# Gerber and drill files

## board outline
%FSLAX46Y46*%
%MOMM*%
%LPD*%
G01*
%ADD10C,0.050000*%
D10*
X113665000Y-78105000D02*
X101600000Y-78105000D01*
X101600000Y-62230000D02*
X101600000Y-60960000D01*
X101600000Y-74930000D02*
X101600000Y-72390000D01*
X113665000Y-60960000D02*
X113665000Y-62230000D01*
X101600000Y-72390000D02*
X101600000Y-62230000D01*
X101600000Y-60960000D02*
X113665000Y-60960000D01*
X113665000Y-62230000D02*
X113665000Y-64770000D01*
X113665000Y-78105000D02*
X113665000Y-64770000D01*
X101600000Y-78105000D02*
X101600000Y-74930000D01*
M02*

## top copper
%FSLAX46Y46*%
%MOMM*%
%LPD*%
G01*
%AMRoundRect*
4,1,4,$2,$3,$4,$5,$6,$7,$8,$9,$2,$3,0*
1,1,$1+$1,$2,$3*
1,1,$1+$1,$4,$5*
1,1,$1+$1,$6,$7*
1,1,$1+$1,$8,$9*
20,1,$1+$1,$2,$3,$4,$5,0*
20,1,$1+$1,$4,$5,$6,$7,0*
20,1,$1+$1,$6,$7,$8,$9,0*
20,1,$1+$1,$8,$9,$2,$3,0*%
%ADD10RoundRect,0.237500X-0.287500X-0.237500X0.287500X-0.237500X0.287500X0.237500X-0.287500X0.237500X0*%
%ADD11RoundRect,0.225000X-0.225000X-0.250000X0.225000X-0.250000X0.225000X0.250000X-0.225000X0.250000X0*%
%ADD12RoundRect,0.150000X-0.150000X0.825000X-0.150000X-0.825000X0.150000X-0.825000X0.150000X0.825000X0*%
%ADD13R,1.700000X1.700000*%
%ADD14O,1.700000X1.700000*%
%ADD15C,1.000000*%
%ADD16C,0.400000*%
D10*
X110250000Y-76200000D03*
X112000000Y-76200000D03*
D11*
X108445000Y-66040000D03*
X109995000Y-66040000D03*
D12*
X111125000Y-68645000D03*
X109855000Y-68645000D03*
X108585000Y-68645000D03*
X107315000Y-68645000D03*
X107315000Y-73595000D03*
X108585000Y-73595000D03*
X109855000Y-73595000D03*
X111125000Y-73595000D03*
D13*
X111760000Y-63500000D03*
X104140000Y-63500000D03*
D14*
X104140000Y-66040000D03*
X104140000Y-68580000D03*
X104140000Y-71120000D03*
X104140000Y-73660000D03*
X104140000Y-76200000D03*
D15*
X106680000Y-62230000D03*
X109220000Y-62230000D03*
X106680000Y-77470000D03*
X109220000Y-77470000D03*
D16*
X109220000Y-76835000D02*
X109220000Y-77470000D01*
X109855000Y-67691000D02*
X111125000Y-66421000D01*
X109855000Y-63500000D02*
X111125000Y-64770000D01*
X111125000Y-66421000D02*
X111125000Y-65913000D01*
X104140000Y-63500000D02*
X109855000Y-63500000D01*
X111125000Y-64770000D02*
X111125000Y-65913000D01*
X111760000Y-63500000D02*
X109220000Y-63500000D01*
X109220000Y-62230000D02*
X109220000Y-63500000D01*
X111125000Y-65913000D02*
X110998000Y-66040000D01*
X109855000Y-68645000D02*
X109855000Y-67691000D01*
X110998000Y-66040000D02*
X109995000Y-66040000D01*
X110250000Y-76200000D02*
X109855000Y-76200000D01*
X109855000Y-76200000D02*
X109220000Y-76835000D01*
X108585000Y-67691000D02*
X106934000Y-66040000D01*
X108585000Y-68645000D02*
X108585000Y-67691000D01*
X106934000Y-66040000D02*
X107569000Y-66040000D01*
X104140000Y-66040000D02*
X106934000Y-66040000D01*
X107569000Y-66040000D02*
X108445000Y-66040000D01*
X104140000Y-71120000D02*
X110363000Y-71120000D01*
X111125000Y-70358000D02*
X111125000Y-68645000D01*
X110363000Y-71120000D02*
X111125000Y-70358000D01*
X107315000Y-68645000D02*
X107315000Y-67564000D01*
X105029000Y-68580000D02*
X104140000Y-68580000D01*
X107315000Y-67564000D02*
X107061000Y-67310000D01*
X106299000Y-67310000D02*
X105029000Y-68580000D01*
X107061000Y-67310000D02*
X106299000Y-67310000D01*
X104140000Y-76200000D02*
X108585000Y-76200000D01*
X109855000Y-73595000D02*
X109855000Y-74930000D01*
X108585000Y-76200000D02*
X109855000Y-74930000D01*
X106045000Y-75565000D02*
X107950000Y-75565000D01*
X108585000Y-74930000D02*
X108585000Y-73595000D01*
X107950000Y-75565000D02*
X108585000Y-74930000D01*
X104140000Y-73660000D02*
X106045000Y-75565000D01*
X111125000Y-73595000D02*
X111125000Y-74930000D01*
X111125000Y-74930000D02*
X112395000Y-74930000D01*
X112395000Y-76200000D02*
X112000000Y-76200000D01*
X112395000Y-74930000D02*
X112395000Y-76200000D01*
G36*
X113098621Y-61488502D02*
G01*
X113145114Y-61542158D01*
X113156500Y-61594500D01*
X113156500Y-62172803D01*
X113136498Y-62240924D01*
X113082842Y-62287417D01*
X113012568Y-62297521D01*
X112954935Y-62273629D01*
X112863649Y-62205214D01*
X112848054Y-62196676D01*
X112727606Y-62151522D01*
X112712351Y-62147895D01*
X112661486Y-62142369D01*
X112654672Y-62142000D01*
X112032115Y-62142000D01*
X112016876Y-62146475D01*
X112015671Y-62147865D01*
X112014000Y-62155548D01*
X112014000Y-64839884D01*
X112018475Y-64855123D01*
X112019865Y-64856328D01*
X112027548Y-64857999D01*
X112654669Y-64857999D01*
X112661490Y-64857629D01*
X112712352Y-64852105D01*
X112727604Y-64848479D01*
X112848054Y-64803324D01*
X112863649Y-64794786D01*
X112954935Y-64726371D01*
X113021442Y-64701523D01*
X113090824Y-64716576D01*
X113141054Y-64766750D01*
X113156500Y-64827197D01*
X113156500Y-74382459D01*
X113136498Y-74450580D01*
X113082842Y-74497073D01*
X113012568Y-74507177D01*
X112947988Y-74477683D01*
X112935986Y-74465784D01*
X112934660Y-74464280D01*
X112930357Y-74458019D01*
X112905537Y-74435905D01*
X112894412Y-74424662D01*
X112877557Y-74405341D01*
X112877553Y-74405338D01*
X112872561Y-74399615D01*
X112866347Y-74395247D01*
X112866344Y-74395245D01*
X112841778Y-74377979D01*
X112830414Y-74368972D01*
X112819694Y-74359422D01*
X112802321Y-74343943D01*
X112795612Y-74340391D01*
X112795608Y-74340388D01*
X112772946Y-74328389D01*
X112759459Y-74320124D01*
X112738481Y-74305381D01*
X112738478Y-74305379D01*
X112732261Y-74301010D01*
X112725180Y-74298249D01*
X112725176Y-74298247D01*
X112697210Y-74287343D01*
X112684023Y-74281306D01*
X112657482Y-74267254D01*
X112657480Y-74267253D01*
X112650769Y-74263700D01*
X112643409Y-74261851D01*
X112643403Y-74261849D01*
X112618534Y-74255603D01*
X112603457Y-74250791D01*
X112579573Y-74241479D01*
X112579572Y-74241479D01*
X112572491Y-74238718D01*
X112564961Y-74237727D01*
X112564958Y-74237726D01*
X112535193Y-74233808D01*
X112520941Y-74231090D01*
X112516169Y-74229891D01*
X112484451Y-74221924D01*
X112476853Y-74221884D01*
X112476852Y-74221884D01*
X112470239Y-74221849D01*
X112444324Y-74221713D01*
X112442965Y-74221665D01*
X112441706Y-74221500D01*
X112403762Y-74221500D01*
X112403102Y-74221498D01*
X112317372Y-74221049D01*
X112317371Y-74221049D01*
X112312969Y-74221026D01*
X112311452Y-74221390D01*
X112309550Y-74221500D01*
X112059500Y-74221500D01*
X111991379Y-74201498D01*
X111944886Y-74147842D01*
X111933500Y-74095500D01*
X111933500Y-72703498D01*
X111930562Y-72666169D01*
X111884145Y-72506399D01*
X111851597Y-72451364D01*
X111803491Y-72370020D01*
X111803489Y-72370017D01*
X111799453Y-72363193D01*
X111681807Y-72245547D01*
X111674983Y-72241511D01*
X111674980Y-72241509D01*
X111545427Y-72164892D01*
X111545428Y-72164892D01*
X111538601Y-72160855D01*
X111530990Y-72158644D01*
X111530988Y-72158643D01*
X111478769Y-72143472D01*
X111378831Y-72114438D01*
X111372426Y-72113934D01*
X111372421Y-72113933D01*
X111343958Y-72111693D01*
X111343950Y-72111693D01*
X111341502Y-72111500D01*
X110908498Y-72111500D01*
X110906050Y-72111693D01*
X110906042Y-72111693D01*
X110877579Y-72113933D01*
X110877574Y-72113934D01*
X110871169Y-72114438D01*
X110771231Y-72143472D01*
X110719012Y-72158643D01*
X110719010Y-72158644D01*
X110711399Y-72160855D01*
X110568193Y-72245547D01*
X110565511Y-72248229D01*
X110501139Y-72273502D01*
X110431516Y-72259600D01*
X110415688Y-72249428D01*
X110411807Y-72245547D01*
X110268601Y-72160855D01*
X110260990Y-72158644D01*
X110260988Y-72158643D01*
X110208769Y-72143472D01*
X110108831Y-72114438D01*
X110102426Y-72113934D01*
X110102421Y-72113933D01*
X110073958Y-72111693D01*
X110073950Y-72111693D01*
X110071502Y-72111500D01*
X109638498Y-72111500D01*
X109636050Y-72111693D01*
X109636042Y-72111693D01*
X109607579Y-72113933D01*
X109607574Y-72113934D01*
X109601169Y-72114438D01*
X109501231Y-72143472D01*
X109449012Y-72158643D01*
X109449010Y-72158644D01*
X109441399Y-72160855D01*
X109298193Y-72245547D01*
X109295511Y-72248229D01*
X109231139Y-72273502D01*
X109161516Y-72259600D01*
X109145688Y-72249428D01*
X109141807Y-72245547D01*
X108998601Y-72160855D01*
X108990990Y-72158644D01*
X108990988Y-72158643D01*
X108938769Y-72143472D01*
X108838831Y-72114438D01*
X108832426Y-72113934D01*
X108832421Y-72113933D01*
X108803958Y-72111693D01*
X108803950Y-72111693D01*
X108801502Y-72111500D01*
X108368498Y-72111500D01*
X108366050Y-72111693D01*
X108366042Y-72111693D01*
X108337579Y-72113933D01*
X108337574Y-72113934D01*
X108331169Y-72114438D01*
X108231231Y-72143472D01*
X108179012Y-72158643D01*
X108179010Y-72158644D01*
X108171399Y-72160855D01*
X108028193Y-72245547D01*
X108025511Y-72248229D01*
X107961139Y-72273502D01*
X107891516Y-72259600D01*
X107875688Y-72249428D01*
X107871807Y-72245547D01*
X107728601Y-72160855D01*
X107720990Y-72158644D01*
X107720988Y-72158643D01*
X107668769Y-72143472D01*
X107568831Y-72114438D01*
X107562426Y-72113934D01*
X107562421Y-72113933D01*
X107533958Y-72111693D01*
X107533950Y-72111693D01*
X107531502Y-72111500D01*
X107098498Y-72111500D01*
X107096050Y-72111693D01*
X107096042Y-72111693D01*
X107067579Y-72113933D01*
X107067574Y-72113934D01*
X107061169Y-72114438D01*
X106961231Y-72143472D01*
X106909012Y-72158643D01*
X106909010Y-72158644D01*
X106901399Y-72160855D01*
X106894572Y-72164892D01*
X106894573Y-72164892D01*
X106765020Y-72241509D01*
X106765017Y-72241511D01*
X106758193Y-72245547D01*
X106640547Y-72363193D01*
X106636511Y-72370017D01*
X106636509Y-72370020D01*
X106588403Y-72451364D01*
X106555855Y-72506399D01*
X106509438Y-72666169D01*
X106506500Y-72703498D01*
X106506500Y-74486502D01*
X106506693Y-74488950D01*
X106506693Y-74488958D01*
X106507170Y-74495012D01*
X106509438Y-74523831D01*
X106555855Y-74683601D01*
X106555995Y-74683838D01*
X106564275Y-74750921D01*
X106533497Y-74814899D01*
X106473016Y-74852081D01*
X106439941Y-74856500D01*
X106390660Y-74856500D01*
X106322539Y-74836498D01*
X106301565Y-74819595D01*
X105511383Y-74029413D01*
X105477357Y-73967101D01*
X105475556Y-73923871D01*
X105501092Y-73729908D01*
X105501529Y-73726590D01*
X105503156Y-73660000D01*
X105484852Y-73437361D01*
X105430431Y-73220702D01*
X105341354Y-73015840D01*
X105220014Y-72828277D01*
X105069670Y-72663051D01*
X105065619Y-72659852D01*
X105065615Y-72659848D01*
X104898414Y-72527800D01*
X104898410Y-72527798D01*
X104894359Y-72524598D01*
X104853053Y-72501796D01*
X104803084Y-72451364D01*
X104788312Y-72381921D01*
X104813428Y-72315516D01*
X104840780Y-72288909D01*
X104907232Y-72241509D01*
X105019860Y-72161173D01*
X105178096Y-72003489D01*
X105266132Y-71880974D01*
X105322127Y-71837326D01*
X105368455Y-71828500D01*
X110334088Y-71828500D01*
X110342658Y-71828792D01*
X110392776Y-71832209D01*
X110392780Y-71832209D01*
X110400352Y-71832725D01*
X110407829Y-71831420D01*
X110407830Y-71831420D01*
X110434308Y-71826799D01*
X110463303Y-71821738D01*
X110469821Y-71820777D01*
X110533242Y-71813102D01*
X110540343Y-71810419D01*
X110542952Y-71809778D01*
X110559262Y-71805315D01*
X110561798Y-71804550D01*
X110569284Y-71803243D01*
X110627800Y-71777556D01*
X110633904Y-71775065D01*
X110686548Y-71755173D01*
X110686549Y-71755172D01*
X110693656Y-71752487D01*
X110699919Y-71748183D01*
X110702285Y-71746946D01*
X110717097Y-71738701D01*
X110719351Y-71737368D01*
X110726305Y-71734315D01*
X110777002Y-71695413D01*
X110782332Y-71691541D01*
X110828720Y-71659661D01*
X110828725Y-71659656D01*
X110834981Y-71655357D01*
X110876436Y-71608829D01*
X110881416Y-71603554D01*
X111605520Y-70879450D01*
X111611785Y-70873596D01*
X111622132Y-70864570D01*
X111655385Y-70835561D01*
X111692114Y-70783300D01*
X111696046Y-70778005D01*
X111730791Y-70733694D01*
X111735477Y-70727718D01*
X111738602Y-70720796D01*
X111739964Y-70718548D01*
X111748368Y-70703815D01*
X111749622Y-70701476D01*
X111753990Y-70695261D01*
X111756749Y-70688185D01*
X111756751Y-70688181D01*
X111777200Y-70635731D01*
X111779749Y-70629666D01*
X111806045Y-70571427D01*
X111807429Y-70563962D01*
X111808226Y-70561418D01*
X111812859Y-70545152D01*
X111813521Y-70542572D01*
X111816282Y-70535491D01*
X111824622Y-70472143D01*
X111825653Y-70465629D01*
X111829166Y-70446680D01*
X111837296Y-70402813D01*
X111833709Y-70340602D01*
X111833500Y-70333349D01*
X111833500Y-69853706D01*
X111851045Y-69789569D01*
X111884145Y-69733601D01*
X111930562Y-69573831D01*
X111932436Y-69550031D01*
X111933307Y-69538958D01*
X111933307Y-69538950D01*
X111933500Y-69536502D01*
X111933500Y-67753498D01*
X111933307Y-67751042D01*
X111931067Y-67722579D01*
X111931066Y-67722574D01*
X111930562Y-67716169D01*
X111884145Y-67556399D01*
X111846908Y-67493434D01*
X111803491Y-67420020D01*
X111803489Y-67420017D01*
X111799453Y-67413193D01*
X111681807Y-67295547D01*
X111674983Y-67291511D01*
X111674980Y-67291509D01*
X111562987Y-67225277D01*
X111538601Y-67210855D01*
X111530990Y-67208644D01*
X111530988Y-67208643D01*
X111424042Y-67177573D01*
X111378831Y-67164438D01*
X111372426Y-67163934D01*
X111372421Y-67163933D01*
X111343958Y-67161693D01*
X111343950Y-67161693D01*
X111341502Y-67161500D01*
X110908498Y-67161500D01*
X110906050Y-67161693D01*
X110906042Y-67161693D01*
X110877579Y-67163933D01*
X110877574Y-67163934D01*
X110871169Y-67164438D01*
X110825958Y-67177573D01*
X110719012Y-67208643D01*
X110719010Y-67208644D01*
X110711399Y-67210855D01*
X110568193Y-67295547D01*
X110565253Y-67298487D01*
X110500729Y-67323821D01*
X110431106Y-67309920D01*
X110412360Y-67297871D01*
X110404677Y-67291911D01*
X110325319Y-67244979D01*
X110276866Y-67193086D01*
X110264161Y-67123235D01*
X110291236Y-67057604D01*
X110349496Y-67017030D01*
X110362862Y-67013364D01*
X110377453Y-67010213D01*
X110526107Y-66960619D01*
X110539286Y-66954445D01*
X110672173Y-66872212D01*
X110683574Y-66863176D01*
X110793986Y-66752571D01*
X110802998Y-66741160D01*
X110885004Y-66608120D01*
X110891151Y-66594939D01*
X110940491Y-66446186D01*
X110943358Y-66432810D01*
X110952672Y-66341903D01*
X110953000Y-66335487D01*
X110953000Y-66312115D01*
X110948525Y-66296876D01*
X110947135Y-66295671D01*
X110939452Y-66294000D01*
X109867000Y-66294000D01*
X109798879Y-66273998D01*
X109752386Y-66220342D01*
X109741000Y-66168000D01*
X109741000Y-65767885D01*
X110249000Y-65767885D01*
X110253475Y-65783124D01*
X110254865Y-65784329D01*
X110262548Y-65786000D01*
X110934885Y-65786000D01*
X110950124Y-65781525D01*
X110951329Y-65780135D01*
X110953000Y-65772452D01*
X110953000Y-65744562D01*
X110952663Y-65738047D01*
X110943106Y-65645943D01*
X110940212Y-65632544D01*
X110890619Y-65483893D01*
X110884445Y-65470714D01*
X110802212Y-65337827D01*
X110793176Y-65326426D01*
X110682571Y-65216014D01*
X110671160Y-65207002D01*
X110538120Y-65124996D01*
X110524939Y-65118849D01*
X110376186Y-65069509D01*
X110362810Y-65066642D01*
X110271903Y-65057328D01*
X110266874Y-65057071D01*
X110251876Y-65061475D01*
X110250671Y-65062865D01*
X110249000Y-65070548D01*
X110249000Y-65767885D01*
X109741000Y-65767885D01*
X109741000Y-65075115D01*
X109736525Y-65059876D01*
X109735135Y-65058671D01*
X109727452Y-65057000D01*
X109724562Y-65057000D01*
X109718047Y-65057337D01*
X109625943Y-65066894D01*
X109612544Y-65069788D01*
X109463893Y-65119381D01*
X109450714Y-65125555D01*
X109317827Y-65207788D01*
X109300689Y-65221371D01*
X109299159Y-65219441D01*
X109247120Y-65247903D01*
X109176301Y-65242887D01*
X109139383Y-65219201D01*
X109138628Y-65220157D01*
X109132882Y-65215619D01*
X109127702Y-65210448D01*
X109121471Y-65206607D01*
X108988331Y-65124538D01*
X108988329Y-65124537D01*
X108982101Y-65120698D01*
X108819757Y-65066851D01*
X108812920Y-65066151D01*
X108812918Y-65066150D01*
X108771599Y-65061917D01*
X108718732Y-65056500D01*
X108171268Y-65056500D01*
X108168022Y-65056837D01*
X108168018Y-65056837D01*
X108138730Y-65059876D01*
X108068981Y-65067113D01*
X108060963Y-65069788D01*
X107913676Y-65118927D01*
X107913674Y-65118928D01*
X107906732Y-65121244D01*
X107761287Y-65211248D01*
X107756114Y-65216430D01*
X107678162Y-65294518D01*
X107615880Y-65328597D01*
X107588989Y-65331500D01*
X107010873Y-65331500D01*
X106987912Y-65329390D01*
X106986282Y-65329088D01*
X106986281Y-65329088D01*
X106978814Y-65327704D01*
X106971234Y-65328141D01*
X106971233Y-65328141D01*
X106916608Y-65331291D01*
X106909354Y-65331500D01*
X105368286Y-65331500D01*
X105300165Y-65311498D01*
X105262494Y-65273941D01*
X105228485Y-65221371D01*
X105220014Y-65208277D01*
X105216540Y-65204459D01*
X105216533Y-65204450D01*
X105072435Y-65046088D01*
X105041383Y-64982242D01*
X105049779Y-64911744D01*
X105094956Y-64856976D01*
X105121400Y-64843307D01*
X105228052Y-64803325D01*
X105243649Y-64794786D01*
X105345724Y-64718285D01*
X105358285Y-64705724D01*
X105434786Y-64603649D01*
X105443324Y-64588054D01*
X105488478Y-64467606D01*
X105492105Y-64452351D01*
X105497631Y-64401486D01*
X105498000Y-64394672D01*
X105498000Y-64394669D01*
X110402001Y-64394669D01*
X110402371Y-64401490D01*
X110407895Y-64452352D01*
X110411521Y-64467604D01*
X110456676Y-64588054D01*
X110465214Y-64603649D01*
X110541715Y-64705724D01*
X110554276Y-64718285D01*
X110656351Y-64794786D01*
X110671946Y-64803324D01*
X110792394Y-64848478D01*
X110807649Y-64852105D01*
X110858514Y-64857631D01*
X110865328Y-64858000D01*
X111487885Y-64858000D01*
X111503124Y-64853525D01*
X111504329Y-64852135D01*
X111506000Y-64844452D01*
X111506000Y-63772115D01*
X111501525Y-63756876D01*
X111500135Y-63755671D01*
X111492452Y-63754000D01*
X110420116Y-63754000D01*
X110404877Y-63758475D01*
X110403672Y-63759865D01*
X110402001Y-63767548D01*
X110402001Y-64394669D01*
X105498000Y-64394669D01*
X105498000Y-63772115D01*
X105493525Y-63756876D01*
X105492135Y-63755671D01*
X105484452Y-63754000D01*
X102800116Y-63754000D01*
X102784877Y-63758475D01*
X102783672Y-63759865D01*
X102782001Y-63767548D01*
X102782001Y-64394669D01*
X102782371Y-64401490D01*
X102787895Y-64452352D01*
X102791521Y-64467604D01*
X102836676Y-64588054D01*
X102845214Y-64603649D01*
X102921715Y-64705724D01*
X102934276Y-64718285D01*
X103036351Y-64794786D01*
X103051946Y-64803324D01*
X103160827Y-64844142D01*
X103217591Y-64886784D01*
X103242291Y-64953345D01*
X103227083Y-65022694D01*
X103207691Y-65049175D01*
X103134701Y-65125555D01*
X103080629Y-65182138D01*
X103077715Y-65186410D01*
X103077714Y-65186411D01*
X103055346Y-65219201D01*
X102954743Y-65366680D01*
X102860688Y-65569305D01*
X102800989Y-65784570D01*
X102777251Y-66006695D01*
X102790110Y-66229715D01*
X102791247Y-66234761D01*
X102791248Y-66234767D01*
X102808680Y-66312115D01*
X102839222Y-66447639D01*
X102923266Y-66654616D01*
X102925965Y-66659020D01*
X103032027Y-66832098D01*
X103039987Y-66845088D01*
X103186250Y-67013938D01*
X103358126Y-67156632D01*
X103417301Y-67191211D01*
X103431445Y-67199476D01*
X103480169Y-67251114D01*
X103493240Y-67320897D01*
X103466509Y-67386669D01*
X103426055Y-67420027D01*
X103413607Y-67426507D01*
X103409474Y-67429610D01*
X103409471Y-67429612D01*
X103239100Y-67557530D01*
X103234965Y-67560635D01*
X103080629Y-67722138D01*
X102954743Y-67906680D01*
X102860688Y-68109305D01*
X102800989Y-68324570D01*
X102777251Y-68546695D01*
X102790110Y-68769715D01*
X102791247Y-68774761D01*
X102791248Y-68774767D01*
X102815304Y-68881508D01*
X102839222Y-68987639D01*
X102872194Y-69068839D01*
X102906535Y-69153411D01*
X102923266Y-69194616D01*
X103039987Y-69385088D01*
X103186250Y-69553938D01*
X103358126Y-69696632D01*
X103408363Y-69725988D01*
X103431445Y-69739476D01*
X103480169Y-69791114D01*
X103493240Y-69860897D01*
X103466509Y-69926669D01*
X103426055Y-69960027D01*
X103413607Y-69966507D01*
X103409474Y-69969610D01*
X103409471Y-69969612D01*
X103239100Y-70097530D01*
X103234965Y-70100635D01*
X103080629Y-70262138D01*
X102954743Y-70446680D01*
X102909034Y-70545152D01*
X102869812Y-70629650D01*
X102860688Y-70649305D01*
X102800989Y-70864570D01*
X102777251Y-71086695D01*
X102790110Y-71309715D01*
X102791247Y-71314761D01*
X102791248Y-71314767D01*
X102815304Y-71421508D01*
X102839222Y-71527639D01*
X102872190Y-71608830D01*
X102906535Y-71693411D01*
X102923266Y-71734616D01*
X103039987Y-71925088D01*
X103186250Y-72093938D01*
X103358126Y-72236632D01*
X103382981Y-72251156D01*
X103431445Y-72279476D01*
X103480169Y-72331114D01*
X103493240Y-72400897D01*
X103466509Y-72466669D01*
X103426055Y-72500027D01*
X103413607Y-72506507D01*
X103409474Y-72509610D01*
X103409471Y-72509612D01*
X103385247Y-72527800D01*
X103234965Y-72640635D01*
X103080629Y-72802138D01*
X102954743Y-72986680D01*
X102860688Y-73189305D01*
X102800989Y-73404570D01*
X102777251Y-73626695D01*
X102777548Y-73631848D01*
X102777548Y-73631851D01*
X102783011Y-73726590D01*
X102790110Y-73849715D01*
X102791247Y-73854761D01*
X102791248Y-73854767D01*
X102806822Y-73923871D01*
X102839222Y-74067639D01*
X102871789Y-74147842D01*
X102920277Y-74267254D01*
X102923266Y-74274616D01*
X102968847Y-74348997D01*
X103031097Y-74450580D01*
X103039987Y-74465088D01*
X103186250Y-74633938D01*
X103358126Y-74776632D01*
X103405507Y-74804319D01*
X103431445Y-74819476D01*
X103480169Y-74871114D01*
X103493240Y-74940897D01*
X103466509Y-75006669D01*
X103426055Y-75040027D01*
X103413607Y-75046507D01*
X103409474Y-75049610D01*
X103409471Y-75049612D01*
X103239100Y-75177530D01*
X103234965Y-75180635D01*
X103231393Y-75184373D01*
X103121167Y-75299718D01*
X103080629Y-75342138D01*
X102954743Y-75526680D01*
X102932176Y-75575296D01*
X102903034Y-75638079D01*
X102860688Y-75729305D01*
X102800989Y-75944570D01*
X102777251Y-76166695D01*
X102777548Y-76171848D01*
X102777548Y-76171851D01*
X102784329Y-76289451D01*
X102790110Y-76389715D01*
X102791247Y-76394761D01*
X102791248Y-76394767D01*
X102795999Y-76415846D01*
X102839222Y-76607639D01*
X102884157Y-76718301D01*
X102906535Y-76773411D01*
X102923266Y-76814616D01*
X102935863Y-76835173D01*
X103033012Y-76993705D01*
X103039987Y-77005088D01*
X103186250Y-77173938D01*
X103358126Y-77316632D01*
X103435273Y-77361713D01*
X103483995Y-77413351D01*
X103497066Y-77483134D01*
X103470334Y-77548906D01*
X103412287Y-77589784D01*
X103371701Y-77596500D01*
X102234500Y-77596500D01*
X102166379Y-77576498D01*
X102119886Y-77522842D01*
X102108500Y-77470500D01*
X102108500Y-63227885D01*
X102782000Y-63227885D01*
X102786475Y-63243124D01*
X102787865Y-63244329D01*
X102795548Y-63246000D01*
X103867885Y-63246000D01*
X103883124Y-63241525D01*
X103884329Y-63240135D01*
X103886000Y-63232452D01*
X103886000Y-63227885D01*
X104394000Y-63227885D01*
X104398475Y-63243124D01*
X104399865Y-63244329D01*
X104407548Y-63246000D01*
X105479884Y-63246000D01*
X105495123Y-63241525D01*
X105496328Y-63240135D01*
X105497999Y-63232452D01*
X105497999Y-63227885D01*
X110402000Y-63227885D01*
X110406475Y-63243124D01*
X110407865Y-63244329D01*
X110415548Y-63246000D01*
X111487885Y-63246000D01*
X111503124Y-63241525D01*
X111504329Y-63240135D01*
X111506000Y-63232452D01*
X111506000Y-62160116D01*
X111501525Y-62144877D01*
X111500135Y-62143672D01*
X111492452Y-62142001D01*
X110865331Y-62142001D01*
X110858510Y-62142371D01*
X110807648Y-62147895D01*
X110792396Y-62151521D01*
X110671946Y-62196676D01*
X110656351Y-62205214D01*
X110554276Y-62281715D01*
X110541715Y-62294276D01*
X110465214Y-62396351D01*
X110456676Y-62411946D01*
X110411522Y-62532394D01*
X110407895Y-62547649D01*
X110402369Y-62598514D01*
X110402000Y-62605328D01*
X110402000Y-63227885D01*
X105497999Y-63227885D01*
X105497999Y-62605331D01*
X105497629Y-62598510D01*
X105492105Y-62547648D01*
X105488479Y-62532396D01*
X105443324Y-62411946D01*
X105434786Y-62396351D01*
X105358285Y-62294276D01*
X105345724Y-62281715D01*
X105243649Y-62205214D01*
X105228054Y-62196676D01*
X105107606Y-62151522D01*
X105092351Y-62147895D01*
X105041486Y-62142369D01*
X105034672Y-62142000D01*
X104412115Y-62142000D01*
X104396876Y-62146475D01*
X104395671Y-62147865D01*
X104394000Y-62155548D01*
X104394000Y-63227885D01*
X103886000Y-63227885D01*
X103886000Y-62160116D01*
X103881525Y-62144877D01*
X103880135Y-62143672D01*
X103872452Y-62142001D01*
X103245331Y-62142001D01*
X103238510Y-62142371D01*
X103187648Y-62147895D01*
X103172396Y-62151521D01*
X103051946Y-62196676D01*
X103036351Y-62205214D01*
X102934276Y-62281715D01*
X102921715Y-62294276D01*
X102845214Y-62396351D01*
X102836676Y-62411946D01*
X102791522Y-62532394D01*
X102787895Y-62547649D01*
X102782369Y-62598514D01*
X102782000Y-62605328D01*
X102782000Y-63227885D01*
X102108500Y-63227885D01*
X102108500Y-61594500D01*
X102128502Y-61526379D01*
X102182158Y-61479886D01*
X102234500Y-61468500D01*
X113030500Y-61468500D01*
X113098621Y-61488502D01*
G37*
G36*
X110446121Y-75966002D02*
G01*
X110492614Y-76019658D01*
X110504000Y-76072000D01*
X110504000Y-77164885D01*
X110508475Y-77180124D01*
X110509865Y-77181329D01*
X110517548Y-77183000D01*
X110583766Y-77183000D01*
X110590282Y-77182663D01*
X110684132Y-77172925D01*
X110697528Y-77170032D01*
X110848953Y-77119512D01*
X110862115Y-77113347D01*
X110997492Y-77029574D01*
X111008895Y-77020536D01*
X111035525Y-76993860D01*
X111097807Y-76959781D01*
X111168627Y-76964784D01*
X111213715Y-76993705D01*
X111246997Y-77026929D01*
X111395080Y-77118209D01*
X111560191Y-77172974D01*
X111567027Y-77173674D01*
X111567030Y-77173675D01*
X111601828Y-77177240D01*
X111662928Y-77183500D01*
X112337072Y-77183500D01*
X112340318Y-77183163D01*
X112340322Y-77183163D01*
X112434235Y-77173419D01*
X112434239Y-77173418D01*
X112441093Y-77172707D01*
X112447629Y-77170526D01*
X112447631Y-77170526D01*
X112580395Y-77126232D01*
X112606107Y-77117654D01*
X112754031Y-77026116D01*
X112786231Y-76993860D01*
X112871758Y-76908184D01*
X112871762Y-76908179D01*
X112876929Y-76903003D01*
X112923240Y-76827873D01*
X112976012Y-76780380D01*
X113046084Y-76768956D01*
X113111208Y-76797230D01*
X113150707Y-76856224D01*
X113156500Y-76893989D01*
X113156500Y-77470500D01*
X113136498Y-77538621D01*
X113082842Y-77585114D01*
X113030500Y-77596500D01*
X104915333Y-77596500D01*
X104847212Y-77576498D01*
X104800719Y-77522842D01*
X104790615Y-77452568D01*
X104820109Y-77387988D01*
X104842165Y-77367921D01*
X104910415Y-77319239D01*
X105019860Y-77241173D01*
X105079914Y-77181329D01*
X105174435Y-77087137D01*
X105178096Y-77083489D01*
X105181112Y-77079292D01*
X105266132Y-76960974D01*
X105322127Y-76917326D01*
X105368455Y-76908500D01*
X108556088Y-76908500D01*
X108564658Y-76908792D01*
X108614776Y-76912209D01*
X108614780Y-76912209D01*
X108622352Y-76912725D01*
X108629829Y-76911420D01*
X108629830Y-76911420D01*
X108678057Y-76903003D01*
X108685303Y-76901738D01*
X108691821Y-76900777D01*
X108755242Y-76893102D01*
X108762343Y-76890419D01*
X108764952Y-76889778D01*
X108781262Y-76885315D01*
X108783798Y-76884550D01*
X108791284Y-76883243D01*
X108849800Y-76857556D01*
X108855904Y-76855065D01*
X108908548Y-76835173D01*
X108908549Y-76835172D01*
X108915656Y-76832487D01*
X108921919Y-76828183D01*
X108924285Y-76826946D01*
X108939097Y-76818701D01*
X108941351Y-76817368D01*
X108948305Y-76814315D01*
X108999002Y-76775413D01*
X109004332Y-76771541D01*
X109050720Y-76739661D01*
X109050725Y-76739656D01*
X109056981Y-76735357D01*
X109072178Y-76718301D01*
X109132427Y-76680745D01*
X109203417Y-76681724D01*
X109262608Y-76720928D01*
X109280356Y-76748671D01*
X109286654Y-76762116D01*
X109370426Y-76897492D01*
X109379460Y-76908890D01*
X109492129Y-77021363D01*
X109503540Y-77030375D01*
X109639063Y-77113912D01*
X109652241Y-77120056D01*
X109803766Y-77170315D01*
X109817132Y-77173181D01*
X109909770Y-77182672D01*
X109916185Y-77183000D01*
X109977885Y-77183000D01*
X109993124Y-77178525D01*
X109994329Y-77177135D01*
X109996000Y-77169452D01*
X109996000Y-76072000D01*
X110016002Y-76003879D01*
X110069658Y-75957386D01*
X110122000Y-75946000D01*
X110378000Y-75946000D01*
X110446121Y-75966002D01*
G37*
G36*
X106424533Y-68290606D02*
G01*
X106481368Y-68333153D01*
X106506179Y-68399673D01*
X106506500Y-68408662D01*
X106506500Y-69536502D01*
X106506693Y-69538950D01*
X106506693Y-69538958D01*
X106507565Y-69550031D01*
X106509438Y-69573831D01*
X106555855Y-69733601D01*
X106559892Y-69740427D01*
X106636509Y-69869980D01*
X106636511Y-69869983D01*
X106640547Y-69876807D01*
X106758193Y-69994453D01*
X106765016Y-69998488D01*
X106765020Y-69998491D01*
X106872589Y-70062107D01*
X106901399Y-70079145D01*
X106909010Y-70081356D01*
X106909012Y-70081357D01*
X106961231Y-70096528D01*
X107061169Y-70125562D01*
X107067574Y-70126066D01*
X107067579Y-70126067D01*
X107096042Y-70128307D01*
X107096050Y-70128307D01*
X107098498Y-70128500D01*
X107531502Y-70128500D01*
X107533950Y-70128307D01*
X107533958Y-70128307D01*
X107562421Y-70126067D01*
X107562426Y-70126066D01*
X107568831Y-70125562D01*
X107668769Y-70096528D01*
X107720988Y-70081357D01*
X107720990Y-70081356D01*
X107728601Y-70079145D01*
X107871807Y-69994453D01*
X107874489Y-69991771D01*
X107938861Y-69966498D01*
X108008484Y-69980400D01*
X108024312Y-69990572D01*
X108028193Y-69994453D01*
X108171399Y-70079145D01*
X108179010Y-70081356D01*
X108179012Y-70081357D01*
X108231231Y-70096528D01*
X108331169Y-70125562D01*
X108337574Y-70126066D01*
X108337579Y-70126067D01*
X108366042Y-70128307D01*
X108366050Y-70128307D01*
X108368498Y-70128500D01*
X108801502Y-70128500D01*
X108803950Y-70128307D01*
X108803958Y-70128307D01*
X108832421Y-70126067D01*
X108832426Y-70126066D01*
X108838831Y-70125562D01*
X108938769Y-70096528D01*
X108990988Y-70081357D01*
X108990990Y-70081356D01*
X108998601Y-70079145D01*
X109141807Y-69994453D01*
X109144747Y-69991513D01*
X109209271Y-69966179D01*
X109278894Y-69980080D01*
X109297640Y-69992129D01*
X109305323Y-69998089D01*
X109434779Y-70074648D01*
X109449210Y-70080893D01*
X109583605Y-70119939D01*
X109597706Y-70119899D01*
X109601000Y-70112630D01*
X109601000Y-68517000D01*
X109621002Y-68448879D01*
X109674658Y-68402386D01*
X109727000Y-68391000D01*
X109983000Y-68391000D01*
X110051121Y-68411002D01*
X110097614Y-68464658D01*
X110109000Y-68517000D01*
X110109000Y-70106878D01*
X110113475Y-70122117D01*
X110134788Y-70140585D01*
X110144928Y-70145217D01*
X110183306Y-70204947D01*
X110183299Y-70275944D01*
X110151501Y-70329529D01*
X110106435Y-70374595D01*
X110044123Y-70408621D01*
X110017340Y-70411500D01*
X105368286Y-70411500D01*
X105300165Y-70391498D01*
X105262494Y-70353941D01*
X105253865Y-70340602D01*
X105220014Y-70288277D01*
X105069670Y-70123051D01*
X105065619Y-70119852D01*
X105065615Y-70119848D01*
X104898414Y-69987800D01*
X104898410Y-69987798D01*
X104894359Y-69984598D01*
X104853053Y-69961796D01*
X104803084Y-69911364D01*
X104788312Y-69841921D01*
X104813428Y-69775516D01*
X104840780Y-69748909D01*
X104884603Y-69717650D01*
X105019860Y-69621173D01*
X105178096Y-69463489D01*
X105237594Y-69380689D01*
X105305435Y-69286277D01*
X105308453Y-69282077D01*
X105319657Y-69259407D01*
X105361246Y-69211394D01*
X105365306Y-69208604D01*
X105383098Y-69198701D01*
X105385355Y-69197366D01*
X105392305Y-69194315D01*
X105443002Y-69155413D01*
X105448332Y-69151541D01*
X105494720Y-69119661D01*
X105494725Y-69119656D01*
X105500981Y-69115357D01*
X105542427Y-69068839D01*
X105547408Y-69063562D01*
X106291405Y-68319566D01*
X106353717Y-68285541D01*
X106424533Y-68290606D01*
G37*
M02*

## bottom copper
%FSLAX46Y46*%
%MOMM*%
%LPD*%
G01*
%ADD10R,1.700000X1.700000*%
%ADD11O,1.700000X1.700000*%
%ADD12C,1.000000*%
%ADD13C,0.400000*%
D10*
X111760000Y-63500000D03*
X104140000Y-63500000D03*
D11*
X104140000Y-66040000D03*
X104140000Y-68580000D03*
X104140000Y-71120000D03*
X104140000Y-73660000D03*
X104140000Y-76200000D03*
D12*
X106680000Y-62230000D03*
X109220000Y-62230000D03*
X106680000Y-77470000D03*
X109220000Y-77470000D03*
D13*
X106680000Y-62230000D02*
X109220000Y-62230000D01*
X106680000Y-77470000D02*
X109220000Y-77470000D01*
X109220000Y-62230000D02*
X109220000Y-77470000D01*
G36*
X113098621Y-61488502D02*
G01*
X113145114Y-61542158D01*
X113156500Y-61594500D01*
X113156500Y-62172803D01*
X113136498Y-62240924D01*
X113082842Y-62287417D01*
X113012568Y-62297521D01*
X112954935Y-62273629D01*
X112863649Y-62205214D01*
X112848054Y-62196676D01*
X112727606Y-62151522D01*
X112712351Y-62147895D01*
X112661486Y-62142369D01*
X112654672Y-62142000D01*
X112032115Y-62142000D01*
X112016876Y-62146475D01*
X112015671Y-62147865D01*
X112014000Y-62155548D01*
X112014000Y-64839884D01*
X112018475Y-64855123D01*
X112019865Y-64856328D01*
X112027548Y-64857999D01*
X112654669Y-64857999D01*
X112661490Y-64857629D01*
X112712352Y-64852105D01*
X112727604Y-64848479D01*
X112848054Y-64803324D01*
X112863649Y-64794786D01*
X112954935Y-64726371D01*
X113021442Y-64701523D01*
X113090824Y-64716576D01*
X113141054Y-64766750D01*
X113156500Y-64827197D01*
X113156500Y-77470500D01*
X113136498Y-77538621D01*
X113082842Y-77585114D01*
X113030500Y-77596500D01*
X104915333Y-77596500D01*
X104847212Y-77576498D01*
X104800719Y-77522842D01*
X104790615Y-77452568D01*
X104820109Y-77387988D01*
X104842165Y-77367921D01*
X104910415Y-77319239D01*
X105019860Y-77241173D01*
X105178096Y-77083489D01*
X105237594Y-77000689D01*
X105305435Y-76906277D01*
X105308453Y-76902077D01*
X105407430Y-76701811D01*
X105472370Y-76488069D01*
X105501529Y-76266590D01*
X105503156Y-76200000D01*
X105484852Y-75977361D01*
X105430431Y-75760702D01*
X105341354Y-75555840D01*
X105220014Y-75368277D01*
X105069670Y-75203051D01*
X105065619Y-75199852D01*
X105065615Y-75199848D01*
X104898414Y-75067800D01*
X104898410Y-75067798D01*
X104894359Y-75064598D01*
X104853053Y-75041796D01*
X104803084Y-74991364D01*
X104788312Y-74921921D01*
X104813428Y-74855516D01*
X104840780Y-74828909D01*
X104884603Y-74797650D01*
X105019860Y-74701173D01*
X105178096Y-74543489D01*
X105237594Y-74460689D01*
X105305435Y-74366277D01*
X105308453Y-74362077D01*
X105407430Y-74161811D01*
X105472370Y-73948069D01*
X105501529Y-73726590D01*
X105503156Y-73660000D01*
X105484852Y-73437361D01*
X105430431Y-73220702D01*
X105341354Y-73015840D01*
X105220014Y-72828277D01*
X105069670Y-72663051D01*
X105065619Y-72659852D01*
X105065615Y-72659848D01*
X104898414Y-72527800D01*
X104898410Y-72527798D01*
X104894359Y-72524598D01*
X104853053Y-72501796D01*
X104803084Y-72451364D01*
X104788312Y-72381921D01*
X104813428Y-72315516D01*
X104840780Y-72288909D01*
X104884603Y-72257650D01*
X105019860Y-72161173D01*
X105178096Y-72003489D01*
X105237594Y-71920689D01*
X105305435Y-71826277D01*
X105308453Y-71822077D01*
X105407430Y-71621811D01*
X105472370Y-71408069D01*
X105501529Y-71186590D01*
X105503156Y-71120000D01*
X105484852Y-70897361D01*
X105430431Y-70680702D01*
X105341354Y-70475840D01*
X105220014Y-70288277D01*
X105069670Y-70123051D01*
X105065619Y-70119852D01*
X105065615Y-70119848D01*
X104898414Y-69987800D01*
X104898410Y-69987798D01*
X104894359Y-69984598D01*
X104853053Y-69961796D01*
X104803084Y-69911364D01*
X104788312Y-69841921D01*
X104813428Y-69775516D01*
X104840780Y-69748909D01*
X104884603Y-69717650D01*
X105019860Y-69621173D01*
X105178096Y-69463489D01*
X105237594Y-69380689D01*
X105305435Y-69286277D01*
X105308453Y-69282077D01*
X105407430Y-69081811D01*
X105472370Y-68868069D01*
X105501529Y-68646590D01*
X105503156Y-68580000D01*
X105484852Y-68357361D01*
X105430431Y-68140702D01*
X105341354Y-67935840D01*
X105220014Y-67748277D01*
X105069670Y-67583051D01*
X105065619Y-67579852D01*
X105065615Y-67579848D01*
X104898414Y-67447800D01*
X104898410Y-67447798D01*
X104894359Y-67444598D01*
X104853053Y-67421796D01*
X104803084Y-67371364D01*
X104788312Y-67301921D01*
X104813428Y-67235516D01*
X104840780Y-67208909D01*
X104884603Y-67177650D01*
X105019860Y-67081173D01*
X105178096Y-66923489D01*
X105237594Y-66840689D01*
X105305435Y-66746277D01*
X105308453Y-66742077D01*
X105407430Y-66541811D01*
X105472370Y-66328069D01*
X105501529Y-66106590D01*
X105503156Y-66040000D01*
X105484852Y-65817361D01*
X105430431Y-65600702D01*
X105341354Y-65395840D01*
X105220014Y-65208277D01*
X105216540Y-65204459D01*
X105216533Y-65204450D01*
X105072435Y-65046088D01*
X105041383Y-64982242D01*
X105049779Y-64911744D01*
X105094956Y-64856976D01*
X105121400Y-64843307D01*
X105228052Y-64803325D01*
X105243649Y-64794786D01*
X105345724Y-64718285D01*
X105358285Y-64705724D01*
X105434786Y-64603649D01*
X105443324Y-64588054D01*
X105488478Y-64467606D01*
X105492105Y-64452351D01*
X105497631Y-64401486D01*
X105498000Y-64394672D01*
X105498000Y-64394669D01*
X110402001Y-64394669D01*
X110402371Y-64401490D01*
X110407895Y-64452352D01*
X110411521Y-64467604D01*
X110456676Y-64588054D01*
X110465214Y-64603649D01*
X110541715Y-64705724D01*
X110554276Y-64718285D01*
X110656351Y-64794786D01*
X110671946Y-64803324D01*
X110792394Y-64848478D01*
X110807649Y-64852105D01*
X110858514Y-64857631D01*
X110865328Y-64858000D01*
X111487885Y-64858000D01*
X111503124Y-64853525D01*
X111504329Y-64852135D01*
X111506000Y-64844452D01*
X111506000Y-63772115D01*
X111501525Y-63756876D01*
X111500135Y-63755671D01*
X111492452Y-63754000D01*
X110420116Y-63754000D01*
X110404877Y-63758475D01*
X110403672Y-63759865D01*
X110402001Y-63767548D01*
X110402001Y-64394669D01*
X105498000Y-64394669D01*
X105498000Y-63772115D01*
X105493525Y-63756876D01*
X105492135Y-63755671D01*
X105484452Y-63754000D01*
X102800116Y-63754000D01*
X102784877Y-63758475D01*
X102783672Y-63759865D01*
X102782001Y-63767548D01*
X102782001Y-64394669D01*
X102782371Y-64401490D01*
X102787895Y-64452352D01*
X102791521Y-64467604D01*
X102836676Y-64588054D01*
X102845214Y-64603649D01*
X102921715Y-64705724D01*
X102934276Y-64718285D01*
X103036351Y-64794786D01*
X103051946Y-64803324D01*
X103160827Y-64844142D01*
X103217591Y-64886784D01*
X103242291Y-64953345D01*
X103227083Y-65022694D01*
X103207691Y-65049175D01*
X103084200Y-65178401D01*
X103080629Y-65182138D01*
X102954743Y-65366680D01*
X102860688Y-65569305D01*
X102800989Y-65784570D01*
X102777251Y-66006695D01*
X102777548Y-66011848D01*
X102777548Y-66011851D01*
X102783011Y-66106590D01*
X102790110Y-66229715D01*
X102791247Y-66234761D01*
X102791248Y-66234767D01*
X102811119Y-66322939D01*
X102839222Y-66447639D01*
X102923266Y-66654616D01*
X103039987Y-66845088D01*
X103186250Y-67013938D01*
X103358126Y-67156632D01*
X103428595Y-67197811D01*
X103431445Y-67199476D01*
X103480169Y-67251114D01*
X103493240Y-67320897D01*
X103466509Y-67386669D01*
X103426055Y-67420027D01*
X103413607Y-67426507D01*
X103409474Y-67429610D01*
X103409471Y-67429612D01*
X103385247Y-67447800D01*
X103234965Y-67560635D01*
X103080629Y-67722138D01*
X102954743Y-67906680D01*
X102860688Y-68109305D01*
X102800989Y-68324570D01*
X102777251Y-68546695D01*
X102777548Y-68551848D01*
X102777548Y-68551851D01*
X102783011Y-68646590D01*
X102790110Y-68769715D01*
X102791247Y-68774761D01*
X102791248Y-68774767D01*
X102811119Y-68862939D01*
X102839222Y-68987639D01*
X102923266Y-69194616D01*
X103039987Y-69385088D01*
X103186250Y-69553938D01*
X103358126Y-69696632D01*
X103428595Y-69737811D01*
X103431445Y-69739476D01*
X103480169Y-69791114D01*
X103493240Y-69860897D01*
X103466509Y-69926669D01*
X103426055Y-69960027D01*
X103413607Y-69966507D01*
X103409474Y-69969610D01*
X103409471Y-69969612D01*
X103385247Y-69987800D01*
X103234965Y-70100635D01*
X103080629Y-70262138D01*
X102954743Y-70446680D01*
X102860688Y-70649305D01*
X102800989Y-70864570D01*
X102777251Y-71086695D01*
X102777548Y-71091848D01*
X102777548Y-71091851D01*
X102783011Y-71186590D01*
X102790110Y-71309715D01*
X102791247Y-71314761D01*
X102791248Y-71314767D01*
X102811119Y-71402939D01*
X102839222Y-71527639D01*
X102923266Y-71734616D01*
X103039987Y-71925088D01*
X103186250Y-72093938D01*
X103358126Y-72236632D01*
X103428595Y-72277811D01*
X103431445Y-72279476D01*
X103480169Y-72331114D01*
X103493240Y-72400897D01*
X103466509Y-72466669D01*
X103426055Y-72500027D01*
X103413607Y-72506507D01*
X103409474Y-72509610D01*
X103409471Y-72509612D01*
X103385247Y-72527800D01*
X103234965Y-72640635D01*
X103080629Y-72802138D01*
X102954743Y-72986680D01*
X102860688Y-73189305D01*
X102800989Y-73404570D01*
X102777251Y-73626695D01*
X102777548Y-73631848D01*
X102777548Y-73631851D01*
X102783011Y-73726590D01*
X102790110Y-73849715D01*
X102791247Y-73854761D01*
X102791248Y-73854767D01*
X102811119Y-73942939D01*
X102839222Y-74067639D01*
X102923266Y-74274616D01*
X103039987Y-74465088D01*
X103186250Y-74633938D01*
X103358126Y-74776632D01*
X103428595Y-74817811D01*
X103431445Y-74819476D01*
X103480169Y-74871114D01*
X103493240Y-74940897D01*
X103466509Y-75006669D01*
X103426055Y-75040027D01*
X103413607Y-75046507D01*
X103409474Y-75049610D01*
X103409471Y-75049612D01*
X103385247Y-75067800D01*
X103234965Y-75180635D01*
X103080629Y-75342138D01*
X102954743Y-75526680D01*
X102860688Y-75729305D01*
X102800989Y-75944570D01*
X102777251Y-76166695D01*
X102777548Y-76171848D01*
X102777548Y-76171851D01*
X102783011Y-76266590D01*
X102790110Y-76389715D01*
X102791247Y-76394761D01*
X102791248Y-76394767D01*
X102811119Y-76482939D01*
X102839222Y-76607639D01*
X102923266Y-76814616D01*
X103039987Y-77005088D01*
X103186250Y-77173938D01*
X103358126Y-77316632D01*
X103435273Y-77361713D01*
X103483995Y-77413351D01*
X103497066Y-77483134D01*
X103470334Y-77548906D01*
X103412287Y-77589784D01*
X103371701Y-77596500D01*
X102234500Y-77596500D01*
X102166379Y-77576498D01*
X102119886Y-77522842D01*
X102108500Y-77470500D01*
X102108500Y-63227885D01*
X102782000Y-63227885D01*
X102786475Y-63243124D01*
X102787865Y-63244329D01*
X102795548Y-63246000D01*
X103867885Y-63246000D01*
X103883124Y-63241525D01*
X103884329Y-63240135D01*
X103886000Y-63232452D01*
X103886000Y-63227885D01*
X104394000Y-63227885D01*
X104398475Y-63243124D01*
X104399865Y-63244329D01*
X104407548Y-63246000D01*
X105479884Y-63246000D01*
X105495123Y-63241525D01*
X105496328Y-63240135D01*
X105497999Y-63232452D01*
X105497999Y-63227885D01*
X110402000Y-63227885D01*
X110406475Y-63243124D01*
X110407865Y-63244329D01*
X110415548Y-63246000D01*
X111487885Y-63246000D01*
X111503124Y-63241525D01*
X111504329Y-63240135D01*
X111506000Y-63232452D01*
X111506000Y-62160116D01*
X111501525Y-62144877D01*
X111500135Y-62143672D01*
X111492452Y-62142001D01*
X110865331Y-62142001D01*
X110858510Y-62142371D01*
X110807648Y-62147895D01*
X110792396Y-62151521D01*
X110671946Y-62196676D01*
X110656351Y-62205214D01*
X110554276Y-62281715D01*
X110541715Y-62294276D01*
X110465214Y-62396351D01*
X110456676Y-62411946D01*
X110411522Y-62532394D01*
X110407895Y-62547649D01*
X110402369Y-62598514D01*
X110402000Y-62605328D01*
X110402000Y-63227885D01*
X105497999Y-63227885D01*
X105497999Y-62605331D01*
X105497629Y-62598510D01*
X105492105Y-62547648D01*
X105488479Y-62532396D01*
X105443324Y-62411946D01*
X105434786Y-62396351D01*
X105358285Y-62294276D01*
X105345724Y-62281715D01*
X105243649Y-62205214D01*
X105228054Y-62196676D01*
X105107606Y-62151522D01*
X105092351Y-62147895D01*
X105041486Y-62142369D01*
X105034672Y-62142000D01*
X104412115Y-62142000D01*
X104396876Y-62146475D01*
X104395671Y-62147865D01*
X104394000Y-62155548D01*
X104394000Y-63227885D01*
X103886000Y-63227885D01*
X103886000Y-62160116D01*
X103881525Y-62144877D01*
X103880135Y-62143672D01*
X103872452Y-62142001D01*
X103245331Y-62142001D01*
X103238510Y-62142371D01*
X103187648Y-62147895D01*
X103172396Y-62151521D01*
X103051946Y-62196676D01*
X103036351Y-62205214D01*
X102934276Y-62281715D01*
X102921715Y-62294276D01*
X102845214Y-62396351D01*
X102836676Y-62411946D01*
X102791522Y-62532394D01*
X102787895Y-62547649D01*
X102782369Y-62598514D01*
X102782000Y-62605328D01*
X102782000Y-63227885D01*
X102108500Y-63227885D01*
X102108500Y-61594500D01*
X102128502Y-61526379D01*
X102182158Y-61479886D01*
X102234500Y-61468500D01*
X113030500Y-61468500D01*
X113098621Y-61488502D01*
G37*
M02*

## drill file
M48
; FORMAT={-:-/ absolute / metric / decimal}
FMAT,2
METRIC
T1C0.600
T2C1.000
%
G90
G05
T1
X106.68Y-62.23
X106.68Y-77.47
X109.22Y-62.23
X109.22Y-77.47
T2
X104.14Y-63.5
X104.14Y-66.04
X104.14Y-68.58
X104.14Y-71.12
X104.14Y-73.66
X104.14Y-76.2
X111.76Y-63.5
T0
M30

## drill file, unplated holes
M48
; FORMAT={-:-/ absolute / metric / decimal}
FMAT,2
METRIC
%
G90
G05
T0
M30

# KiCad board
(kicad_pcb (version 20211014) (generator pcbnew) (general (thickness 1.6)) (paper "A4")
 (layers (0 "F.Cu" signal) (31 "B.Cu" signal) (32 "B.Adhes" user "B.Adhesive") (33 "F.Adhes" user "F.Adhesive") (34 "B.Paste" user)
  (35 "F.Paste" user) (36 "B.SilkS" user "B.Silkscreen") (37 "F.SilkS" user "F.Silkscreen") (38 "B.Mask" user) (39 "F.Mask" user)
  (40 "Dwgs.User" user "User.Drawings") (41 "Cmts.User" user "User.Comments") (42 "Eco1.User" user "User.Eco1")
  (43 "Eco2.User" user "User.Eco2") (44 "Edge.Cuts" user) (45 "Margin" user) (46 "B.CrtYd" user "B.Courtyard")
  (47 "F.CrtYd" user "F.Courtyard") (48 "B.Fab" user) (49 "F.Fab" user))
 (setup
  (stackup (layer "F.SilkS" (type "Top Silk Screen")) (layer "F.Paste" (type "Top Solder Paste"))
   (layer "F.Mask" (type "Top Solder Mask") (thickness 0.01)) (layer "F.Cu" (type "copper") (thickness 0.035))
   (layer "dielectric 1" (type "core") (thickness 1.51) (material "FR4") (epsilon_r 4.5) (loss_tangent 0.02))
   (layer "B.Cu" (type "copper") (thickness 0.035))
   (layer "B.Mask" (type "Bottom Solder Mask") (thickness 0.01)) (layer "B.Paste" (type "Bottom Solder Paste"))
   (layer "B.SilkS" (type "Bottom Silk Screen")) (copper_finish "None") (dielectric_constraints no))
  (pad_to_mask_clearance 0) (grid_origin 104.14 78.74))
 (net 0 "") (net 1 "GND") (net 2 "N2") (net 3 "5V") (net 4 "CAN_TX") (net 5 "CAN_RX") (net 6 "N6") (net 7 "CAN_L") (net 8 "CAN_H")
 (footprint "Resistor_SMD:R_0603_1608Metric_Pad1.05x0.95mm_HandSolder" (layer "F.Cu") (at 111.125 76.2)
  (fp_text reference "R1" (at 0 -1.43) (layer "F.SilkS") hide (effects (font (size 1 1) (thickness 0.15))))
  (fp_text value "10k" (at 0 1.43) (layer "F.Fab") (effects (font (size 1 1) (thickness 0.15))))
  (pad "1" smd roundrect locked (at -0.875 0) (size 1.05 0.95) (layers "F.Cu" "F.Paste" "F.Mask") (roundrect_rratio 0.25) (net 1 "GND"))
  (pad "2" smd roundrect locked (at 0.875 0) (size 1.05 0.95) (layers "F.Cu" "F.Paste" "F.Mask") (roundrect_rratio 0.25) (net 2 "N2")))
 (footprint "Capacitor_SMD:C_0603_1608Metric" (layer "F.Cu") (at 109.22 66.04)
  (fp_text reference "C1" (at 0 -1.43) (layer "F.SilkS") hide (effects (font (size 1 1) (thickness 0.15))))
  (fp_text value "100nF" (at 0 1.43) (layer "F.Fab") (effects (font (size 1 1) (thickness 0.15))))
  (pad "1" smd roundrect locked (at -0.775 0) (size 0.9 0.95) (layers "F.Cu" "F.Paste" "F.Mask") (roundrect_rratio 0.25) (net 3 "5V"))
  (pad "2" smd roundrect locked (at 0.775 0) (size 0.9 0.95) (layers "F.Cu" "F.Paste" "F.Mask") (roundrect_rratio 0.25) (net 1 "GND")))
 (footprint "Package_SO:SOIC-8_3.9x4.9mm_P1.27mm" (layer "F.Cu") (at 109.22 71.12 -90)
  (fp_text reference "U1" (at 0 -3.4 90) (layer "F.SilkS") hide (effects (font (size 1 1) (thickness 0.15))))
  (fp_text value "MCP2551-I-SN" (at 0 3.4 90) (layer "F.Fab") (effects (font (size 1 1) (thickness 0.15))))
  (pad "1" smd roundrect locked (at -2.475 -1.905 270) (size 1.95 0.6) (layers "F.Cu" "F.Paste" "F.Mask") (roundrect_rratio 0.25)
   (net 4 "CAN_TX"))
  (pad "2" smd roundrect locked (at -2.475 -0.635 270) (size 1.95 0.6) (layers "F.Cu" "F.Paste" "F.Mask") (roundrect_rratio 0.25)
   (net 1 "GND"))
  (pad "3" smd roundrect locked (at -2.475 0.635 270) (size 1.95 0.6) (layers "F.Cu" "F.Paste" "F.Mask") (roundrect_rratio 0.25)
   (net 3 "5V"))
  (pad "4" smd roundrect locked (at -2.475 1.905 270) (size 1.95 0.6) (layers "F.Cu" "F.Paste" "F.Mask") (roundrect_rratio 0.25)
   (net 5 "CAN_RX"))
  (pad "5" smd roundrect locked (at 2.475 1.905 270) (size 1.95 0.6) (layers "F.Cu" "F.Paste" "F.Mask") (roundrect_rratio 0.25) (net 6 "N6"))
  (pad "6" smd roundrect locked (at 2.475 0.635 270) (size 1.95 0.6) (layers "F.Cu" "F.Paste" "F.Mask") (roundrect_rratio 0.25)
   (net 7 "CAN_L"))
  (pad "7" smd roundrect locked (at 2.475 -0.635 270) (size 1.95 0.6) (layers "F.Cu" "F.Paste" "F.Mask") (roundrect_rratio 0.25)
   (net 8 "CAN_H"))
  (pad "8" smd roundrect locked (at 2.475 -1.905 270) (size 1.95 0.6) (layers "F.Cu" "F.Paste" "F.Mask") (roundrect_rratio 0.25)
   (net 2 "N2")))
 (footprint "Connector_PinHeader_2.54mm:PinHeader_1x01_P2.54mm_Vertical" (layer "B.Cu") (at 111.76 63.5 180)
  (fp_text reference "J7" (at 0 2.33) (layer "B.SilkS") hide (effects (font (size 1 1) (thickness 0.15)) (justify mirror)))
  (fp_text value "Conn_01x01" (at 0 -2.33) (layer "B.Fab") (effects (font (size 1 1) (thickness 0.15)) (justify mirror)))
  (pad "1" thru_hole rect (at 0 0 180) (size 1.7 1.7) (drill 1) (layers *.Cu *.Mask) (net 1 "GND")))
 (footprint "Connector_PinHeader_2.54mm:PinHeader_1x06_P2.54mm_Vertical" (layer "B.Cu") (at 104.14 63.5 180)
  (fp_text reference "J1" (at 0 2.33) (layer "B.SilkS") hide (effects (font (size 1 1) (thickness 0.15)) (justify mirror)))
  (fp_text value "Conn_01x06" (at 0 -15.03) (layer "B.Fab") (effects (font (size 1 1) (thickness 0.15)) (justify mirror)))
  (pad "1" thru_hole rect (at 0 0 180) (size 1.7 1.7) (drill 1) (layers *.Cu *.Mask) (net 1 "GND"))
  (pad "2" thru_hole oval (at 0 -2.54 180) (size 1.7 1.7) (drill 1) (layers *.Cu *.Mask) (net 3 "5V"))
  (pad "3" thru_hole oval (at 0 -5.08 180) (size 1.7 1.7) (drill 1) (layers *.Cu *.Mask) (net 5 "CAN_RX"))
  (pad "4" thru_hole oval (at 0 -7.62 180) (size 1.7 1.7) (drill 1) (layers *.Cu *.Mask) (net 4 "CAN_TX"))
  (pad "5" thru_hole oval (at 0 -10.16 180) (size 1.7 1.7) (drill 1) (layers *.Cu *.Mask) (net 7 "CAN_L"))
  (pad "6" thru_hole oval (at 0 -12.7 180) (size 1.7 1.7) (drill 1) (layers *.Cu *.Mask) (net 8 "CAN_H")))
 (gr_line (start 113.665 78.105) (end 101.6 78.105) (layer "Edge.Cuts") (width 0.05))
 (gr_line (start 101.6 62.23) (end 101.6 60.96) (layer "Edge.Cuts") (width 0.05))
 (gr_line (start 101.6 74.93) (end 101.6 72.39) (layer "Edge.Cuts") (width 0.05))
 (gr_line (start 113.665 60.96) (end 113.665 62.23) (layer "Edge.Cuts") (width 0.05))
 (gr_line (start 101.6 72.39) (end 101.6 62.23) (layer "Edge.Cuts") (width 0.05))
 (gr_line (start 101.6 60.96) (end 113.665 60.96) (layer "Edge.Cuts") (width 0.05))
 (gr_line (start 113.665 62.23) (end 113.665 64.77) (layer "Edge.Cuts") (width 0.05))
 (gr_line (start 113.665 78.105) (end 113.665 64.77) (layer "Edge.Cuts") (width 0.05))
 (gr_line (start 101.6 78.105) (end 101.6 74.93) (layer "Edge.Cuts") (width 0.05))
 (segment (start 109.22 76.835) (end 109.22 77.47) (width 0.4) (layer "F.Cu") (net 1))
 (segment (start 109.855 67.691) (end 111.125 66.421) (width 0.4) (layer "F.Cu") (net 1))
 (segment (start 109.855 63.5) (end 111.125 64.77) (width 0.4) (layer "F.Cu") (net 1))
 (segment (start 111.125 66.421) (end 111.125 65.913) (width 0.4) (layer "F.Cu") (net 1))
 (segment (start 104.14 63.5) (end 109.855 63.5) (width 0.4) (layer "F.Cu") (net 1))
 (segment (start 111.125 64.77) (end 111.125 65.913) (width 0.4) (layer "F.Cu") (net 1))
 (segment (start 111.76 63.5) (end 109.22 63.5) (width 0.4) (layer "F.Cu") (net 1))
 (segment (start 109.22 62.23) (end 109.22 63.5) (width 0.4) (layer "F.Cu") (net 1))
 (segment (start 111.125 65.913) (end 110.998 66.04) (width 0.4) (layer "F.Cu") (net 1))
 (segment (start 109.855 68.645) (end 109.855 67.691) (width 0.4) (layer "F.Cu") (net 1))
 (segment (start 110.998 66.04) (end 109.995 66.04) (width 0.4) (layer "F.Cu") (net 1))
 (segment (start 110.25 76.2) (end 109.855 76.2) (width 0.4) (layer "F.Cu") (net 1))
 (segment (start 109.855 76.2) (end 109.22 76.835) (width 0.4) (layer "F.Cu") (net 1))
 (via (at 106.68 62.23) (size 1) (drill 0.6) (layers "F.Cu" "B.Cu") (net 1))
 (via (at 109.22 62.23) (size 1) (drill 0.6) (layers "F.Cu" "B.Cu") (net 1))
 (via (at 106.68 77.47) (size 1) (drill 0.6) (layers "F.Cu" "B.Cu") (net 1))
 (via (at 109.22 77.47) (size 1) (drill 0.6) (layers "F.Cu" "B.Cu") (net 1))
 (segment (start 106.68 62.23) (end 109.22 62.23) (width 0.4) (layer "B.Cu") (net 1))
 (segment (start 106.68 77.47) (end 109.22 77.47) (width 0.4) (layer "B.Cu") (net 1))
 (segment (start 109.22 62.23) (end 109.22 77.47) (width 0.4) (layer "B.Cu") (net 1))
 (segment (start 108.585 67.691) (end 106.934 66.04) (width 0.4) (layer "F.Cu") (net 3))
 (segment (start 108.585 68.645) (end 108.585 67.691) (width 0.4) (layer "F.Cu") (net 3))
 (segment (start 106.934 66.04) (end 107.569 66.04) (width 0.4) (layer "F.Cu") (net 3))
 (segment (start 104.14 66.04) (end 106.934 66.04) (width 0.4) (layer "F.Cu") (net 3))
 (segment (start 107.569 66.04) (end 108.445 66.04) (width 0.4) (layer "F.Cu") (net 3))
 (segment (start 104.14 71.12) (end 110.363 71.12) (width 0.4) (layer "F.Cu") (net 4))
 (segment (start 111.125 70.358) (end 111.125 68.645) (width 0.4) (layer "F.Cu") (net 4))
 (segment (start 110.363 71.12) (end 111.125 70.358) (width 0.4) (layer "F.Cu") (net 4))
 (segment (start 107.315 68.645) (end 107.315 67.564) (width 0.4) (layer "F.Cu") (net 5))
 (segment (start 105.029 68.58) (end 104.14 68.58) (width 0.4) (layer "F.Cu") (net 5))
 (segment (start 107.315 67.564) (end 107.061 67.31) (width 0.4) (layer "F.Cu") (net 5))
 (segment (start 106.299 67.31) (end 105.029 68.58) (width 0.4) (layer "F.Cu") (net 5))
 (segment (start 107.061 67.31) (end 106.299 67.31) (width 0.4) (layer "F.Cu") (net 5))
 (segment (start 104.14 76.2) (end 108.585 76.2) (width 0.4) (layer "F.Cu") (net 8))
 (segment (start 109.855 73.595) (end 109.855 74.93) (width 0.4) (layer "F.Cu") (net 8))
 (segment (start 108.585 76.2) (end 109.855 74.93) (width 0.4) (layer "F.Cu") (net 8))
 (segment (start 106.045 75.565) (end 107.95 75.565) (width 0.4) (layer "F.Cu") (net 7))
 (segment (start 108.585 74.93) (end 108.585 73.595) (width 0.4) (layer "F.Cu") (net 7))
 (segment (start 107.95 75.565) (end 108.585 74.93) (width 0.4) (layer "F.Cu") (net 7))
 (segment (start 104.14 73.66) (end 106.045 75.565) (width 0.4) (layer "F.Cu") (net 7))
 (segment (start 111.125 73.595) (end 111.125 74.93) (width 0.4) (layer "F.Cu") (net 2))
 (segment (start 111.125 74.93) (end 112.395 74.93) (width 0.4) (layer "F.Cu") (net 2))
 (segment (start 112.395 76.2) (end 112 76.2) (width 0.4) (layer "F.Cu") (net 2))
 (segment (start 112.395 74.93) (end 112.395 76.2) (width 0.4) (layer "F.Cu") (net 2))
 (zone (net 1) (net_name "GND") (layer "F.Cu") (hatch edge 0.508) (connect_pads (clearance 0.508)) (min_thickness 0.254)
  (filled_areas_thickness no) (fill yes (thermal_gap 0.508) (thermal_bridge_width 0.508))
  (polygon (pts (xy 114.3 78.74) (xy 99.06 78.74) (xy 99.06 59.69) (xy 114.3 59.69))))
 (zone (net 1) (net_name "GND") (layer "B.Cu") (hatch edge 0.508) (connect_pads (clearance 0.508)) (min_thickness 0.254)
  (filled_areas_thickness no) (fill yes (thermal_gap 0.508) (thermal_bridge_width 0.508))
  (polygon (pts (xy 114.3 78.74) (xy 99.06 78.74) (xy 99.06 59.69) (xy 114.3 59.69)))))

